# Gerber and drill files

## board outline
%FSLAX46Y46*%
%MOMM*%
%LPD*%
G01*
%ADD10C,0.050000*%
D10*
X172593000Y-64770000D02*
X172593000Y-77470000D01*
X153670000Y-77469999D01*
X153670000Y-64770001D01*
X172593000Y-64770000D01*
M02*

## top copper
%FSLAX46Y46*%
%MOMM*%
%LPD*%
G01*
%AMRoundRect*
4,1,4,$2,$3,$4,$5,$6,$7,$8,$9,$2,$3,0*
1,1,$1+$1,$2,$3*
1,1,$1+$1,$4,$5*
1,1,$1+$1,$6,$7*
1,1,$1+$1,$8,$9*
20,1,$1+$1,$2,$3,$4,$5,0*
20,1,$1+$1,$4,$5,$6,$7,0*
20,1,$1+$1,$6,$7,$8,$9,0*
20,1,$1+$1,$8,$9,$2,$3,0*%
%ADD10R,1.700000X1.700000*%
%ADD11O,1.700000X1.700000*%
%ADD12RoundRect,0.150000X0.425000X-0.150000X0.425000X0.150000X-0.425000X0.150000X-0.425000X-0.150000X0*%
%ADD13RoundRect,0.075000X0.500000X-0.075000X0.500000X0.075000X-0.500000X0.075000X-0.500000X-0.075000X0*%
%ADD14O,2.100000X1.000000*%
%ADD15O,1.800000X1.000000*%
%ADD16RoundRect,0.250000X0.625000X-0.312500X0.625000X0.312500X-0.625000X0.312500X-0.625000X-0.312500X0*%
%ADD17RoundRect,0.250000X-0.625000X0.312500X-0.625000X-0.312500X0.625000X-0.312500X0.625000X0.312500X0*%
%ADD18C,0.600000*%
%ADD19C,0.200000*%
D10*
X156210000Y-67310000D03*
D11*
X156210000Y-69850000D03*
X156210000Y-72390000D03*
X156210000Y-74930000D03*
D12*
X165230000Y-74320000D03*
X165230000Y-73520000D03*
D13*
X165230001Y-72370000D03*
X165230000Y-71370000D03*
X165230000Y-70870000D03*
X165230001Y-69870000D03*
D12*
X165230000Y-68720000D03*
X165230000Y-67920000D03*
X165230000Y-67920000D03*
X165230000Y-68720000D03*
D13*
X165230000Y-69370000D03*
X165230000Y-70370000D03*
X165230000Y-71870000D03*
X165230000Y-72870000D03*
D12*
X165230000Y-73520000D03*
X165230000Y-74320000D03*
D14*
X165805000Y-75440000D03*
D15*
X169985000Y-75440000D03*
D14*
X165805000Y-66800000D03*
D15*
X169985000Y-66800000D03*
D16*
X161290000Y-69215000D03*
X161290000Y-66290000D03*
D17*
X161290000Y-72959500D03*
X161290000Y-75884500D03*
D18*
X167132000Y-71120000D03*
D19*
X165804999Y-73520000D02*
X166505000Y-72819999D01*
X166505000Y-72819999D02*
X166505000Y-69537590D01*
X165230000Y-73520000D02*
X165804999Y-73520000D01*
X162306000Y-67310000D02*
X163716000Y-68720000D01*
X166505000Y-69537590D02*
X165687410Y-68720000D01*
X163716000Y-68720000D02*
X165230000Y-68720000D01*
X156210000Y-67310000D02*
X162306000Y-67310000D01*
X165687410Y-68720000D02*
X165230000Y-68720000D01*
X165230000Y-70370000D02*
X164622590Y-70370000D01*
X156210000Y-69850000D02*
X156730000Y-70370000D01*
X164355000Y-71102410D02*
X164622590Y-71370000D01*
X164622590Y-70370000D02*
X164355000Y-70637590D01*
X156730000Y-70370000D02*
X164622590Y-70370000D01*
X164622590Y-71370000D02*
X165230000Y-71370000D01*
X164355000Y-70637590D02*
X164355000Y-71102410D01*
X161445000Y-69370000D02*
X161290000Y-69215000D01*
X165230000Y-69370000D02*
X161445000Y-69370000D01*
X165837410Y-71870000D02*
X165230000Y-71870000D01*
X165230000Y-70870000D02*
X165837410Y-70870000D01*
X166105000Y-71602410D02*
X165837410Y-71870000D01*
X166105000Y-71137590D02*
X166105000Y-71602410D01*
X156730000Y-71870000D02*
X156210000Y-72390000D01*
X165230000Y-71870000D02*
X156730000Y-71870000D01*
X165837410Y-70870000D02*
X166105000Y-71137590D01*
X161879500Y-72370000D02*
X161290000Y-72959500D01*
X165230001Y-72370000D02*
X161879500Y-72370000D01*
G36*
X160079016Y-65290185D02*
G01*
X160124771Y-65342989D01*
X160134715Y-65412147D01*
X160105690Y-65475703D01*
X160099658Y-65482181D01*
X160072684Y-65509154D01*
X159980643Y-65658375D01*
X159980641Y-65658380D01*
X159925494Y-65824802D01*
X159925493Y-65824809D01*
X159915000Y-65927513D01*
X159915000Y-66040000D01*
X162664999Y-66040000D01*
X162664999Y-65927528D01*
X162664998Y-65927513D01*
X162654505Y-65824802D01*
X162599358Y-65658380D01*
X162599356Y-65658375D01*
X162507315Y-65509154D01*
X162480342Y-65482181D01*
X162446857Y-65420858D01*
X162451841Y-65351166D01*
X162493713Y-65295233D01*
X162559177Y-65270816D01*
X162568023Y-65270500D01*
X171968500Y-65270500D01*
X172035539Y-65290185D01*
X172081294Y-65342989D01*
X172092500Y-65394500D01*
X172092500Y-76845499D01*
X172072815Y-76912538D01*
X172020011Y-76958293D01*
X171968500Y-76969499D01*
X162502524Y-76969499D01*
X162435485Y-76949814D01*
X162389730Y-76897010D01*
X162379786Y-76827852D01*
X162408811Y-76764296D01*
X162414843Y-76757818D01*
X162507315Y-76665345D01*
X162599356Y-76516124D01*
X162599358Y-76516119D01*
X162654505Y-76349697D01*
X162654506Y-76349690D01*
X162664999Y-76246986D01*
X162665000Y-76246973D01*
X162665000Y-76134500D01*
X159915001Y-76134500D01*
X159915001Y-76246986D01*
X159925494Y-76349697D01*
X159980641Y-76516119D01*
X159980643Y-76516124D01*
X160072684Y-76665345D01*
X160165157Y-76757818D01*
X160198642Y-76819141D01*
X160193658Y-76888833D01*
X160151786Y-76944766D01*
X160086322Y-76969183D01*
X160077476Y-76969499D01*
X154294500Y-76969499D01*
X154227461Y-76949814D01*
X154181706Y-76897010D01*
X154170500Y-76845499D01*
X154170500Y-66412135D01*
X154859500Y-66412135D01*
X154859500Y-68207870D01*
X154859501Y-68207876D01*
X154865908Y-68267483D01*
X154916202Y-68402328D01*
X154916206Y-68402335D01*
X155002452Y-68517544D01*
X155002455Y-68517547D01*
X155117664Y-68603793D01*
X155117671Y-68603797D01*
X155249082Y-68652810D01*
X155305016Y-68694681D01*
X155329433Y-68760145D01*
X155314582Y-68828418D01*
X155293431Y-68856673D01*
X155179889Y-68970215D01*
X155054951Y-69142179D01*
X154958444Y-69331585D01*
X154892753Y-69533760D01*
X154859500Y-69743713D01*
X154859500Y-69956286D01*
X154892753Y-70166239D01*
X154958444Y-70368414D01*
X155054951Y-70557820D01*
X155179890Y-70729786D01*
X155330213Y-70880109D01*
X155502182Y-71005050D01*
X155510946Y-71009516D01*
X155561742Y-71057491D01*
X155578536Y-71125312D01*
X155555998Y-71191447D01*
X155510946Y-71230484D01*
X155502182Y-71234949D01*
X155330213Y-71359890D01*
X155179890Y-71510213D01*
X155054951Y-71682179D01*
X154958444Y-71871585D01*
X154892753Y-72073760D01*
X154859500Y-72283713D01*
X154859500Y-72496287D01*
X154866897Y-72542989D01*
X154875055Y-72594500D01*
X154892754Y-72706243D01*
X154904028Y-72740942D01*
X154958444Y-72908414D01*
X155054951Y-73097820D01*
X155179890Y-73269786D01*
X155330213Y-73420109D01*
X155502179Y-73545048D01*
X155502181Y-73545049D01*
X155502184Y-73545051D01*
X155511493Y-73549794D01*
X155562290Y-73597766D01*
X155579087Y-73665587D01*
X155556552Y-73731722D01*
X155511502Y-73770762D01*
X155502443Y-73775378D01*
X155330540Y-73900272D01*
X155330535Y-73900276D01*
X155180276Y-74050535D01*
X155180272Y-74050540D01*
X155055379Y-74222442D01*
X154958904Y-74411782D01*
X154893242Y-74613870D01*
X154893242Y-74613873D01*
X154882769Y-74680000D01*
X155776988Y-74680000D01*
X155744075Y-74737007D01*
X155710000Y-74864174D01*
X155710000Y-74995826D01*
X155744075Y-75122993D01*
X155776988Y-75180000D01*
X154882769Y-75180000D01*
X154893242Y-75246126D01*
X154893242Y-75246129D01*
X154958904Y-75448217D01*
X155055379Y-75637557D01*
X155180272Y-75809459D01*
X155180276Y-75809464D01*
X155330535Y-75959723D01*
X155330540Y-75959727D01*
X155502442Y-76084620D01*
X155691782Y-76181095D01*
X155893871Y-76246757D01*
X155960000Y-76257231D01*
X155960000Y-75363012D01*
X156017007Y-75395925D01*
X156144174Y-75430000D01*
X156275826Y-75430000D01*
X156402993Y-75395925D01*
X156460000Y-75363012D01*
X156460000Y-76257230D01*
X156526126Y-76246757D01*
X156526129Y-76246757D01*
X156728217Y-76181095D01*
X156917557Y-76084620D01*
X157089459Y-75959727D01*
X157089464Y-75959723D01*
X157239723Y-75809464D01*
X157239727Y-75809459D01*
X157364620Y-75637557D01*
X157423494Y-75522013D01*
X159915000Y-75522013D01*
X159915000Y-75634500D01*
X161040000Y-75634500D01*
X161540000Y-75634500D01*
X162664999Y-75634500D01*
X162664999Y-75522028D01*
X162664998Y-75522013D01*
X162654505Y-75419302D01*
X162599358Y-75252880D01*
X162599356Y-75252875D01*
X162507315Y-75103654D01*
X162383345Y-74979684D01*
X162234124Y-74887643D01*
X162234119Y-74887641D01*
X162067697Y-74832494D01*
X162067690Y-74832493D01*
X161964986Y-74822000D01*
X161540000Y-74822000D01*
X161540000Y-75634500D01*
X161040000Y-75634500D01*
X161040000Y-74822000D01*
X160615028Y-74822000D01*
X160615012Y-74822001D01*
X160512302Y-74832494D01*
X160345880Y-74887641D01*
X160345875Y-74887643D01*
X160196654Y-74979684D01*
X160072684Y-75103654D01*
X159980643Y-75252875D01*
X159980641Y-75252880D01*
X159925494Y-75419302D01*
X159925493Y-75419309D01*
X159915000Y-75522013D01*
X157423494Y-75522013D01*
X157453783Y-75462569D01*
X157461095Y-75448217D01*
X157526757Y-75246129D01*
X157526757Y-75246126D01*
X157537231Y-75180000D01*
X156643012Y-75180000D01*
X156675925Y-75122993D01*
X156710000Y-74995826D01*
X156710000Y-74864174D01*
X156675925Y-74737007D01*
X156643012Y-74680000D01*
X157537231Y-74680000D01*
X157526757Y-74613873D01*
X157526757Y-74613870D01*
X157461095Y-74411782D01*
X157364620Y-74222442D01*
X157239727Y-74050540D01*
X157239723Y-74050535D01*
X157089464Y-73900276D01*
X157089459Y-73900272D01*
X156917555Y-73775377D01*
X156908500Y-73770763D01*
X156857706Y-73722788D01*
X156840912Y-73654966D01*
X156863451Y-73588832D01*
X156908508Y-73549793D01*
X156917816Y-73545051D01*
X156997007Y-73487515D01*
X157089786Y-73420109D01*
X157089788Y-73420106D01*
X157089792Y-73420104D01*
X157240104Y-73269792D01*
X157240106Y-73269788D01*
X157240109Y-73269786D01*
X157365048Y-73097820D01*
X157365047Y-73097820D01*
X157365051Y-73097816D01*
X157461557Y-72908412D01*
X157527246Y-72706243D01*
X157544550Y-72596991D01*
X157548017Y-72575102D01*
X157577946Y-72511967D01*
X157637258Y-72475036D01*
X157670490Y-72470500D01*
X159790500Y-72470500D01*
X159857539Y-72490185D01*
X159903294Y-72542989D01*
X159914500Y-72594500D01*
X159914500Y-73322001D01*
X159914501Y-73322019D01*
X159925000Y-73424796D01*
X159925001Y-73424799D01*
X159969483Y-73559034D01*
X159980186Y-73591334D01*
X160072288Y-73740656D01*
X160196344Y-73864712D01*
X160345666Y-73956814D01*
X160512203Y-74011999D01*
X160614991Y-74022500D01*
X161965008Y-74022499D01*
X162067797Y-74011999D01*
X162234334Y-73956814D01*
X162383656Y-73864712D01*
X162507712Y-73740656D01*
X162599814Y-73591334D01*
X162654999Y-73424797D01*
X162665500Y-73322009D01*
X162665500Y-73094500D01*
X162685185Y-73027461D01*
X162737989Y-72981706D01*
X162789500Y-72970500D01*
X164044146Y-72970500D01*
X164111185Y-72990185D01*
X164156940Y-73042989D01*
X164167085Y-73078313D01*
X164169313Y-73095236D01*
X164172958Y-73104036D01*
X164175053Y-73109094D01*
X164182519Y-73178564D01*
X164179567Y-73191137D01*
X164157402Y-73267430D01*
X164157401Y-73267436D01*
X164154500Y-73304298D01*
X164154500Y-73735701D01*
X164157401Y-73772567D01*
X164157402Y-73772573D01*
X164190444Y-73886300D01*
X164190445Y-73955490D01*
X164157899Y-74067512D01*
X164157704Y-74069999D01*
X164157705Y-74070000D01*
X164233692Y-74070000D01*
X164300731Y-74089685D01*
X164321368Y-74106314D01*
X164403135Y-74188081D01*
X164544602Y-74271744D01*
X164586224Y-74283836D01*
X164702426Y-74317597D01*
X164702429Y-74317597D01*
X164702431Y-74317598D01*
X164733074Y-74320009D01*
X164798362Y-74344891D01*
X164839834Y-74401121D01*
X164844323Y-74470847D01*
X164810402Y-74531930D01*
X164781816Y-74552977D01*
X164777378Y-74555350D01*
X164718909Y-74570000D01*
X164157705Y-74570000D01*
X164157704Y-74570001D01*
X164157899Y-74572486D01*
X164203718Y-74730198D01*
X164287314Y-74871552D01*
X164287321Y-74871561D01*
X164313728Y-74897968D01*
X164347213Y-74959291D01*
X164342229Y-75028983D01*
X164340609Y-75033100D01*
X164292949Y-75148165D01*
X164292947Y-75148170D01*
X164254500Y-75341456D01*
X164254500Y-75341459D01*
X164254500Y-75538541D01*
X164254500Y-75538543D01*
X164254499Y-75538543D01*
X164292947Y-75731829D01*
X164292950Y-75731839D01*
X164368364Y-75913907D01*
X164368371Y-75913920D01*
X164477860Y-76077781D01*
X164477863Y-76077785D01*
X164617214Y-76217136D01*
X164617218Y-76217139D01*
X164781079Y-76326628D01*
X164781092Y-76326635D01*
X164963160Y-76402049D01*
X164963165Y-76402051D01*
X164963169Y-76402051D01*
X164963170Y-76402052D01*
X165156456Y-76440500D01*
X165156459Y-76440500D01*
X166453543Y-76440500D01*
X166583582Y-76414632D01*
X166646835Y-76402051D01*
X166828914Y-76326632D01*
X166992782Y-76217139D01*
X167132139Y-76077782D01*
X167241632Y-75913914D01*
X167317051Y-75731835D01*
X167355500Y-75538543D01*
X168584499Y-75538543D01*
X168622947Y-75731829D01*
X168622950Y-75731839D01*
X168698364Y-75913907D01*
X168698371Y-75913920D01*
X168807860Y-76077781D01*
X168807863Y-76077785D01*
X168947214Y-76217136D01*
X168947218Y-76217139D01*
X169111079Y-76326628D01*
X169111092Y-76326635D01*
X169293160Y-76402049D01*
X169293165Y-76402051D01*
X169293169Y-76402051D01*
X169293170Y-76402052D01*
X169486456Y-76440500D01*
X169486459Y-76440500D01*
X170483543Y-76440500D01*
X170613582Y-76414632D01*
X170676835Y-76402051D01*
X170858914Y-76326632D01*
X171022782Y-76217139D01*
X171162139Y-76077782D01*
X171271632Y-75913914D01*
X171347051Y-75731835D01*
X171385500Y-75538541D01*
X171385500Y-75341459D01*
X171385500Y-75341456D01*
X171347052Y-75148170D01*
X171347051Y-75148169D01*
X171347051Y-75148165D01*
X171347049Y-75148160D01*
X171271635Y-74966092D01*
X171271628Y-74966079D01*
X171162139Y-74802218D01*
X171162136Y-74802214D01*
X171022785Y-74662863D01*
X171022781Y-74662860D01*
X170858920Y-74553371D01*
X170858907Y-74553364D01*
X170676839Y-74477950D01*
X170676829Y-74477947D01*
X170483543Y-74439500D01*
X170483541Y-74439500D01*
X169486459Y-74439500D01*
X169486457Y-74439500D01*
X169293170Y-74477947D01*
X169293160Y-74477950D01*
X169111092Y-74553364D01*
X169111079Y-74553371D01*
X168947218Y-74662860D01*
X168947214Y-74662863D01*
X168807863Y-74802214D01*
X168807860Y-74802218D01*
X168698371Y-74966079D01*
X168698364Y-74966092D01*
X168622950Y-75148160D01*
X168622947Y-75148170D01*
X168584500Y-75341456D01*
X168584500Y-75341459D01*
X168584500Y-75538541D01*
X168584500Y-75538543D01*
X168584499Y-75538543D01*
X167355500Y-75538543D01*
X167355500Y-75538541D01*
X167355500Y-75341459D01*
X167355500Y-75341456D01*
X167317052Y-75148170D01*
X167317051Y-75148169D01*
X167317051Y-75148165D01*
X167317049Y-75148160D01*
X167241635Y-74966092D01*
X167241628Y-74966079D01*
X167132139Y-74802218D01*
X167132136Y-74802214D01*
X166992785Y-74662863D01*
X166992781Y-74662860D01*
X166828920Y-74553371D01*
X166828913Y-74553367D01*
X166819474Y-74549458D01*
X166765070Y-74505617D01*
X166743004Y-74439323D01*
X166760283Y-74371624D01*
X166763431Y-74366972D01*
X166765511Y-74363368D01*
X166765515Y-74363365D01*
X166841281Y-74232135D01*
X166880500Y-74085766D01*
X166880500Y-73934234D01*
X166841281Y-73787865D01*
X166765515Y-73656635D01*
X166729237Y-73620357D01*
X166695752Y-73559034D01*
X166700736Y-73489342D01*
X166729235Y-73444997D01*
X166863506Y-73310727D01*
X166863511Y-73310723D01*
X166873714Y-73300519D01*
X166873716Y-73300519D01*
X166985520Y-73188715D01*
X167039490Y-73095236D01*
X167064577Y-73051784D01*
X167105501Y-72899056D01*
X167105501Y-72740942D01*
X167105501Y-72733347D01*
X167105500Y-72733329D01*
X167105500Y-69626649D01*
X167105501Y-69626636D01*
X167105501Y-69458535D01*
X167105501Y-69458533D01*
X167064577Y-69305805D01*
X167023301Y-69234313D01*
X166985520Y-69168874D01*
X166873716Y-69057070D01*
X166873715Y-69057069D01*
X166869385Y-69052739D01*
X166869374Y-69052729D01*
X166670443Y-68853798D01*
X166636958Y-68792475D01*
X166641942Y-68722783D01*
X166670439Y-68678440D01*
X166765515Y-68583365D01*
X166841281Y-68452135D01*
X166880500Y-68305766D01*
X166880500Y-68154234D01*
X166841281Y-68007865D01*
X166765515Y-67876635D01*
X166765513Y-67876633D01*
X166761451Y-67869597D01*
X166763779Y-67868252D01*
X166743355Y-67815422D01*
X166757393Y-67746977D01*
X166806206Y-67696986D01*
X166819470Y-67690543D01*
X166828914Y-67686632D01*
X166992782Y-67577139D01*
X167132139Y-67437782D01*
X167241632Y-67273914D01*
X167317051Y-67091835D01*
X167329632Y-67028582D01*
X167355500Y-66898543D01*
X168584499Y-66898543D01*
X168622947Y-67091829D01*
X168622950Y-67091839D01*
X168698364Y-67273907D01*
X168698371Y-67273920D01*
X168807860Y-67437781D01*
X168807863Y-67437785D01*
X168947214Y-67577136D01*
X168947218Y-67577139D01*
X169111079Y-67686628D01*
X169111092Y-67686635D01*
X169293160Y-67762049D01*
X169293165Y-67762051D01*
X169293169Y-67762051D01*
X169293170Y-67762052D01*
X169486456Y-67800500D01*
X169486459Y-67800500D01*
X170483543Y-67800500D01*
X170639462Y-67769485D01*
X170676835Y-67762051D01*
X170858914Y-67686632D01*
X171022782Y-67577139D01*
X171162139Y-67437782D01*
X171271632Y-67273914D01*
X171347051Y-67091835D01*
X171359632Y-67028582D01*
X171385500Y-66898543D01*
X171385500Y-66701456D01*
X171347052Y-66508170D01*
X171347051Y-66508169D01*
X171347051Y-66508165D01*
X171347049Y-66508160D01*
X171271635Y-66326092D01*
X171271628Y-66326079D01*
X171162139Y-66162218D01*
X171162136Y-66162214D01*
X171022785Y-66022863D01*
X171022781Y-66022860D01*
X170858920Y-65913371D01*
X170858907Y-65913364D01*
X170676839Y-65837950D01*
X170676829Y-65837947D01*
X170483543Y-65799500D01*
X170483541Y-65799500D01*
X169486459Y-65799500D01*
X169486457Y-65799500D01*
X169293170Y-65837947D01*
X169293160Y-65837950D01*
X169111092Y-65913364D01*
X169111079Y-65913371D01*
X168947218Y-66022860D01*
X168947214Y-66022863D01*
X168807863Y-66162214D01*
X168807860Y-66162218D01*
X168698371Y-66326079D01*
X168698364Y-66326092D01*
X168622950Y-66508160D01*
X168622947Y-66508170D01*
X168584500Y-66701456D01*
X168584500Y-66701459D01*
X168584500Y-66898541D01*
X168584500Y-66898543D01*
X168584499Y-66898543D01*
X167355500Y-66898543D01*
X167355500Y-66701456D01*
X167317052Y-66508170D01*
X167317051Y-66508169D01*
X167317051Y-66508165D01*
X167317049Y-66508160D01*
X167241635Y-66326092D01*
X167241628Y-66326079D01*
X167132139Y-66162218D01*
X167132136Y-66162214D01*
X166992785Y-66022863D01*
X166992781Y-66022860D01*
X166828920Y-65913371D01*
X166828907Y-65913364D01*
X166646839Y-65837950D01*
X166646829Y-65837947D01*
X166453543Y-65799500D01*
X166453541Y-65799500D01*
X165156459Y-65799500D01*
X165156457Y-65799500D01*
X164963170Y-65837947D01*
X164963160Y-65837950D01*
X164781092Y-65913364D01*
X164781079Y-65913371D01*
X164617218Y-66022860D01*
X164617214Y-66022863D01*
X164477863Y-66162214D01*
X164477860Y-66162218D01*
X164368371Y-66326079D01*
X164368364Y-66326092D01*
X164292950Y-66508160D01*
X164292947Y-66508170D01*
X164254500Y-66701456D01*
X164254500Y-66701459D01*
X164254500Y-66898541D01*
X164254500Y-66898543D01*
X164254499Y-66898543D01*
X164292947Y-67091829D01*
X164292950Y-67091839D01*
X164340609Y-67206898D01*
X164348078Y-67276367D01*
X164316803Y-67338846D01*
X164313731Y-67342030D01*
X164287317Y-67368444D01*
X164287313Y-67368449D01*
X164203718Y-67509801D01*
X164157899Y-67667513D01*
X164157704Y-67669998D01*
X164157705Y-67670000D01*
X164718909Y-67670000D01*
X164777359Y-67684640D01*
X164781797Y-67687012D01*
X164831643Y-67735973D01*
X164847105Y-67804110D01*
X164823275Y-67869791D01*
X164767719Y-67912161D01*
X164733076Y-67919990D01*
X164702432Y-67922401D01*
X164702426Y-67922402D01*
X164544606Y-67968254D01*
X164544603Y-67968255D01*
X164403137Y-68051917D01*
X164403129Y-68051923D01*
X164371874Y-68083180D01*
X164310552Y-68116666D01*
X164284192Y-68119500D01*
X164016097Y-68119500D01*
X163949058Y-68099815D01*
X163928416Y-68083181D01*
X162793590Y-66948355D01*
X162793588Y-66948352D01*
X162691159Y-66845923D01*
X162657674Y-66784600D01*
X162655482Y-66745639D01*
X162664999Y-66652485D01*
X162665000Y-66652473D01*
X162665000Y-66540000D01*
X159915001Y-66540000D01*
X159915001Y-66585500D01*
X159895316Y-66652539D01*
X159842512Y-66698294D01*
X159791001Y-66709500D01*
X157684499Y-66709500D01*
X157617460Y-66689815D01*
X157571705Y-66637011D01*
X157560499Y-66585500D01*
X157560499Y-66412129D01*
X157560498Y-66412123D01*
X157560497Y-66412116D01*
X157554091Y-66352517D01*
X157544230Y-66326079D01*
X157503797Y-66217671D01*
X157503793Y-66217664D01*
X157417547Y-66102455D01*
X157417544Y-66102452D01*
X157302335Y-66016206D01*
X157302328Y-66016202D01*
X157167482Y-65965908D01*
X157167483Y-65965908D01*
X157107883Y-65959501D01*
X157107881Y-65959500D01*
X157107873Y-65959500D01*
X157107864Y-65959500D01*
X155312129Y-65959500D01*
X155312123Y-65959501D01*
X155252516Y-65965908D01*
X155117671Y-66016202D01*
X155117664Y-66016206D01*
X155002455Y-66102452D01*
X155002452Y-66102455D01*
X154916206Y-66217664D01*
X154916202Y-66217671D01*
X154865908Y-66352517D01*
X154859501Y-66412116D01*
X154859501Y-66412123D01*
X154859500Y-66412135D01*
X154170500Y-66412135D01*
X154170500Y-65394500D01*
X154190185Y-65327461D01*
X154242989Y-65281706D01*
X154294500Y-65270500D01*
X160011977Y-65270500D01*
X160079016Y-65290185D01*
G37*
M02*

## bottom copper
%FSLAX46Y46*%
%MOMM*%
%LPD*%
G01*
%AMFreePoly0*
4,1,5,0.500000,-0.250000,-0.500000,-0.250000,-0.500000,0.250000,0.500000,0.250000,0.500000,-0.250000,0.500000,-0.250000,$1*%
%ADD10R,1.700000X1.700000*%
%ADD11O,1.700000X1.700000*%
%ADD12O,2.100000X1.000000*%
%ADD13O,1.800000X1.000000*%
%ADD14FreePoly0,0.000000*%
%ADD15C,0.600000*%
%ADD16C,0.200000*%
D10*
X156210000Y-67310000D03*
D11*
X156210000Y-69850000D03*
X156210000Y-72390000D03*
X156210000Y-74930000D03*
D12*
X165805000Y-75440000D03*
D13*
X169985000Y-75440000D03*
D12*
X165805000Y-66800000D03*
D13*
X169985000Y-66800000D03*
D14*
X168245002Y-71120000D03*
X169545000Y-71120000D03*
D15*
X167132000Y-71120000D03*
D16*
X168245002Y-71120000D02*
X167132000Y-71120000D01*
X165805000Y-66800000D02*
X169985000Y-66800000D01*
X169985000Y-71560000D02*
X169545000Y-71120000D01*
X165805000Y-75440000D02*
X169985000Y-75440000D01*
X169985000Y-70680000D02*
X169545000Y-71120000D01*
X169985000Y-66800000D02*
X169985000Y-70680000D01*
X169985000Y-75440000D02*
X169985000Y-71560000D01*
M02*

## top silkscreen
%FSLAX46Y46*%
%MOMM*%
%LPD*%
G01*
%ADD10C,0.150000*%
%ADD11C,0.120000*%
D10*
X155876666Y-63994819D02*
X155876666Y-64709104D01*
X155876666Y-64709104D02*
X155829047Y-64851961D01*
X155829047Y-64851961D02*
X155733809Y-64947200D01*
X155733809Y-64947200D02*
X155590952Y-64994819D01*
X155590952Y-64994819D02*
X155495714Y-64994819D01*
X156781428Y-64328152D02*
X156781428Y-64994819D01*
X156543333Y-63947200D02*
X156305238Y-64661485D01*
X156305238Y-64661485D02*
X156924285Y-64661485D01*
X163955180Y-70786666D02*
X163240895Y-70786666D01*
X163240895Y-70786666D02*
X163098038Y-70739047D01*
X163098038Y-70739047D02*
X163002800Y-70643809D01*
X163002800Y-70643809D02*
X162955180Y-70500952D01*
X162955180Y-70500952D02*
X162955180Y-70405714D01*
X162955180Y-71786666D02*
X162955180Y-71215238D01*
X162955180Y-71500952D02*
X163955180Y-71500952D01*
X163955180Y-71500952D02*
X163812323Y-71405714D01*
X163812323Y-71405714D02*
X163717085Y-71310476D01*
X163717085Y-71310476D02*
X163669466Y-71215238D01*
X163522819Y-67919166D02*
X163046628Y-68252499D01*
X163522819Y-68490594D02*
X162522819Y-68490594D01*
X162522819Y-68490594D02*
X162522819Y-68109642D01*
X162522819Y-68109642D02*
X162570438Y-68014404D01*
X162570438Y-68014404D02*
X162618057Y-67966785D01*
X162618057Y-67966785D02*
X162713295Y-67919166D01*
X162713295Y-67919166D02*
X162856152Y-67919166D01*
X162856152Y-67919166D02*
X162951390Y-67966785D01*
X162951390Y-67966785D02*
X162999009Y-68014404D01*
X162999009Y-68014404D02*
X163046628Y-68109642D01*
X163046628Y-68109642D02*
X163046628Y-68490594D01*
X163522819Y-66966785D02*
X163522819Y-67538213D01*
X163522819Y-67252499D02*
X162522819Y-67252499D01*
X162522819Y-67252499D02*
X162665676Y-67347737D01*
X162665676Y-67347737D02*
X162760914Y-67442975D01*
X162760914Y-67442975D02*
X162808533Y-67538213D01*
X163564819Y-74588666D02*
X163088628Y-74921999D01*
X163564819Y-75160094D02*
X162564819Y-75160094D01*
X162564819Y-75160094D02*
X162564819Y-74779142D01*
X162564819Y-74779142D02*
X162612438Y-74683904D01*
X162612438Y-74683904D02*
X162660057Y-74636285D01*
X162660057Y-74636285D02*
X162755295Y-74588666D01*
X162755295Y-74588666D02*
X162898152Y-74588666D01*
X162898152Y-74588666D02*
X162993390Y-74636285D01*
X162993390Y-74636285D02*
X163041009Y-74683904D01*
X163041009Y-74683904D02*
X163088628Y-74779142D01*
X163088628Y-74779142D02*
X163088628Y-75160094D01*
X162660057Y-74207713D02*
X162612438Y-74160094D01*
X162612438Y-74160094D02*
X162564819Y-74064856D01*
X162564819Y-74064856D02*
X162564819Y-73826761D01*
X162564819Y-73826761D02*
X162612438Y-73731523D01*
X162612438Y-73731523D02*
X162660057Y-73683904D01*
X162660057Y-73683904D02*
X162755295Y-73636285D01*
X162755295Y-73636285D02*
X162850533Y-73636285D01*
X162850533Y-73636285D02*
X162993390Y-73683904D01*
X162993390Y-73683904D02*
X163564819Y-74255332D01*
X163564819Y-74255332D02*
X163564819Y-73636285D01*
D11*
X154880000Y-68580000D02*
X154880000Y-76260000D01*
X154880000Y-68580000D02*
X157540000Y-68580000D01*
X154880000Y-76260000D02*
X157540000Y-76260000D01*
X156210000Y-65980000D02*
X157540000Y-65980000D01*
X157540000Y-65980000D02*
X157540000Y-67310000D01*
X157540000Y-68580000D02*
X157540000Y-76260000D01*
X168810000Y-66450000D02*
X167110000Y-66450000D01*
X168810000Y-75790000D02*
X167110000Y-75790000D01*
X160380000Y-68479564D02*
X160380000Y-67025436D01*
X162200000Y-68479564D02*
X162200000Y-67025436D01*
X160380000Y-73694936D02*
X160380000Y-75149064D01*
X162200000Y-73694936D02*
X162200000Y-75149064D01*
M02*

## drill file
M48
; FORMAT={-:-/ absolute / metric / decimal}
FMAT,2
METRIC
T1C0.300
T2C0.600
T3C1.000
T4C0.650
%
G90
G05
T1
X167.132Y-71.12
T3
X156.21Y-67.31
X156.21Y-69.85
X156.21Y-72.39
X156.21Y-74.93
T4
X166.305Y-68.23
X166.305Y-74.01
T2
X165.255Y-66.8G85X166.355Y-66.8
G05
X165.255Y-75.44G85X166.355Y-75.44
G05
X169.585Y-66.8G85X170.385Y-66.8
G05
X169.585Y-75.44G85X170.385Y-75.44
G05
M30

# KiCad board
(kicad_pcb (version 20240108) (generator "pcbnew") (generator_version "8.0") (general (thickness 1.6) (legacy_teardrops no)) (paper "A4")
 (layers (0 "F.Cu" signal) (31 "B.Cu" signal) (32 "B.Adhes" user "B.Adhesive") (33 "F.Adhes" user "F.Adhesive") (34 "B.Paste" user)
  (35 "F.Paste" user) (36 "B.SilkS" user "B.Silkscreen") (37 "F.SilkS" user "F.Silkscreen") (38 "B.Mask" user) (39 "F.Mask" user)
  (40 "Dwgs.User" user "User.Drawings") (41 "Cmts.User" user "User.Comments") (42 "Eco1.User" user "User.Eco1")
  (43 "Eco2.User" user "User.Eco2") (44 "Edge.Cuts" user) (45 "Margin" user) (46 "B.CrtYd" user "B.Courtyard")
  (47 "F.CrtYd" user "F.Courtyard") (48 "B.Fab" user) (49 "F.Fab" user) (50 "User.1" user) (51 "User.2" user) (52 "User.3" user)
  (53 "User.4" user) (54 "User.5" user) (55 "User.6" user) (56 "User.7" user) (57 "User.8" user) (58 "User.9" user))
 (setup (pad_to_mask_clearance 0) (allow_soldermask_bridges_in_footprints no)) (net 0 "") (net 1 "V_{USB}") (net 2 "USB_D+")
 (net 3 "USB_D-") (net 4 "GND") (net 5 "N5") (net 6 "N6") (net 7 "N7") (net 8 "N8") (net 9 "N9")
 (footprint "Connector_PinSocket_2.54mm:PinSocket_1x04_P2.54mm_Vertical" (layer "F.Cu") (at 156.21 67.31)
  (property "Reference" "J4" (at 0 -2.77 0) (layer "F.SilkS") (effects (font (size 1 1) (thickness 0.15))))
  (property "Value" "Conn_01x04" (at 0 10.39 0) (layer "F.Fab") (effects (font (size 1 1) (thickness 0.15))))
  (fp_line (start -1.33 1.27) (end -1.33 8.95) (stroke (width 0.12) (type solid)) (layer "F.SilkS"))
  (fp_line (start -1.33 1.27) (end 1.33 1.27) (stroke (width 0.12) (type solid)) (layer "F.SilkS"))
  (fp_line (start -1.33 8.95) (end 1.33 8.95) (stroke (width 0.12) (type solid)) (layer "F.SilkS"))
  (fp_line (start 0 -1.33) (end 1.33 -1.33) (stroke (width 0.12) (type solid)) (layer "F.SilkS"))
  (fp_line (start 1.33 -1.33) (end 1.33 0) (stroke (width 0.12) (type solid)) (layer "F.SilkS"))
  (fp_line (start 1.33 1.27) (end 1.33 8.95) (stroke (width 0.12) (type solid)) (layer "F.SilkS"))
  (pad "1" thru_hole rect (at 0 0) (size 1.7 1.7) (drill 1) (layers "*.Cu" "*.Mask") (remove_unused_layers no) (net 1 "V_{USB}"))
  (pad "2" thru_hole oval (at 0 2.54) (size 1.7 1.7) (drill 1) (layers "*.Cu" "*.Mask") (remove_unused_layers no) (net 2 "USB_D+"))
  (pad "3" thru_hole oval (at 0 5.08) (size 1.7 1.7) (drill 1) (layers "*.Cu" "*.Mask") (remove_unused_layers no) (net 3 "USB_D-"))
  (pad "4" thru_hole oval (at 0 7.62) (size 1.7 1.7) (drill 1) (layers "*.Cu" "*.Mask") (remove_unused_layers no) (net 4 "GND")))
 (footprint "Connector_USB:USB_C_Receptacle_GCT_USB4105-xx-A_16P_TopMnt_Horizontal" (layer "F.Cu") (at 168.91 71.12 90)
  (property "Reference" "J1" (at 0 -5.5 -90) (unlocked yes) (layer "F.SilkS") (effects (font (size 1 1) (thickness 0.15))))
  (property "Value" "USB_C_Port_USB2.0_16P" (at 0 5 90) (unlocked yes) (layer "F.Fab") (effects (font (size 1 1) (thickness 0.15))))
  (fp_line (start 4.67 -0.1) (end 4.67 -1.8) (stroke (width 0.12) (type solid)) (layer "F.SilkS"))
  (fp_line (start -4.67 -0.1) (end -4.67 -1.8) (stroke (width 0.12) (type solid)) (layer "F.SilkS"))
  (pad "" np_thru_hole circle (at -2.89 -2.605 90) (size 0.65 0.65) (drill 0.65) (layers "F&B.Cu" "*.Mask"))
  (pad "" np_thru_hole circle (at 2.89 -2.605 90) (size 0.65 0.65) (drill 0.65) (layers "F&B.Cu" "*.Mask"))
  (pad "A1" smd roundrect (at -3.2 -3.68 90) (size 0.6 1.15) (layers "F.Cu" "F.Paste" "F.Mask") (roundrect_rratio 0.25) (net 4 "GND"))
  (pad "A4" smd roundrect (at -2.4 -3.68 90) (size 0.6 1.15) (layers "F.Cu" "F.Paste" "F.Mask") (roundrect_rratio 0.25) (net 1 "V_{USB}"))
  (pad "A5" smd roundrect (at -1.25 -3.679999 90) (size 0.3 1.15) (layers "F.Cu" "F.Paste" "F.Mask") (roundrect_rratio 0.25) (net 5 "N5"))
  (pad "A6" smd roundrect (at -0.25 -3.68 90) (size 0.3 1.15) (layers "F.Cu" "F.Paste" "F.Mask") (roundrect_rratio 0.25) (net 2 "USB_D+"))
  (pad "A7" smd roundrect (at 0.25 -3.68 90) (size 0.3 1.15) (layers "F.Cu" "F.Paste" "F.Mask") (roundrect_rratio 0.25) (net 3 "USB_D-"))
  (pad "A8" smd roundrect (at 1.25 -3.679999 90) (size 0.3 1.15) (layers "F.Cu" "F.Paste" "F.Mask") (roundrect_rratio 0.25) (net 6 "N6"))
  (pad "A9" smd roundrect (at 2.4 -3.68 90) (size 0.6 1.15) (layers "F.Cu" "F.Paste" "F.Mask") (roundrect_rratio 0.25) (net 1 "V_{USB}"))
  (pad "A12" smd roundrect (at 3.2 -3.68 90) (size 0.6 1.15) (layers "F.Cu" "F.Paste" "F.Mask") (roundrect_rratio 0.25) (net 4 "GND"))
  (pad "B1" smd roundrect (at 3.2 -3.68 90) (size 0.6 1.15) (layers "F.Cu" "F.Paste" "F.Mask") (roundrect_rratio 0.25) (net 4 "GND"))
  (pad "B4" smd roundrect (at 2.4 -3.68 90) (size 0.6 1.15) (layers "F.Cu" "F.Paste" "F.Mask") (roundrect_rratio 0.25) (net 1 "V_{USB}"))
  (pad "B5" smd roundrect (at 1.75 -3.68 90) (size 0.3 1.15) (layers "F.Cu" "F.Paste" "F.Mask") (roundrect_rratio 0.25) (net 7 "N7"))
  (pad "B6" smd roundrect (at 0.75 -3.68 90) (size 0.3 1.15) (layers "F.Cu" "F.Paste" "F.Mask") (roundrect_rratio 0.25) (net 2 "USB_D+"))
  (pad "B7" smd roundrect (at -0.75 -3.68 90) (size 0.3 1.15) (layers "F.Cu" "F.Paste" "F.Mask") (roundrect_rratio 0.25) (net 3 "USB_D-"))
  (pad "B8" smd roundrect (at -1.75 -3.68 90) (size 0.3 1.15) (layers "F.Cu" "F.Paste" "F.Mask") (roundrect_rratio 0.25) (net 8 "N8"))
  (pad "B9" smd roundrect (at -2.4 -3.68 90) (size 0.6 1.15) (layers "F.Cu" "F.Paste" "F.Mask") (roundrect_rratio 0.25) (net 1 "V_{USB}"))
  (pad "B12" smd roundrect (at -3.2 -3.68 90) (size 0.6 1.15) (layers "F.Cu" "F.Paste" "F.Mask") (roundrect_rratio 0.25) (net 4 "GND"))
  (pad "S1" thru_hole oval (at -4.32 -3.105 90) (size 1 2.1) (drill oval 0.6 1.7) (layers "*.Cu" "*.Mask" "F.Paste")
   (remove_unused_layers no) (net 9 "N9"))
  (pad "S1" thru_hole oval (at -4.32 1.075 90) (size 1 1.8) (drill oval 0.6 1.4) (layers "*.Cu" "*.Mask" "F.Paste")
   (remove_unused_layers no) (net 9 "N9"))
  (pad "S1" thru_hole oval (at 4.32 -3.105 90) (size 1 2.1) (drill oval 0.6 1.7) (layers "*.Cu" "*.Mask" "F.Paste")
   (remove_unused_layers no) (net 9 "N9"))
  (pad "S1" thru_hole oval (at 4.32 1.075 90) (size 1 1.8) (drill oval 0.6 1.4) (layers "*.Cu" "*.Mask" "F.Paste") (remove_unused_layers no)
   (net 9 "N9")))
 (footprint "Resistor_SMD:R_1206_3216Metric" (layer "F.Cu") (at 161.29 67.7525 90)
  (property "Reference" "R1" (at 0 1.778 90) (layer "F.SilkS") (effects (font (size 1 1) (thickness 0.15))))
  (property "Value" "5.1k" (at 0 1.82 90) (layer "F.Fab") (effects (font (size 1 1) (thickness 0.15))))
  (fp_line (start -0.727064 -0.91) (end 0.727064 -0.91) (stroke (width 0.12) (type solid)) (layer "F.SilkS"))
  (fp_line (start -0.727064 0.91) (end 0.727064 0.91) (stroke (width 0.12) (type solid)) (layer "F.SilkS"))
  (pad "1" smd roundrect (at -1.4625 0 90) (size 1.125 1.75) (layers "F.Cu" "F.Paste" "F.Mask") (roundrect_rratio 0.222222) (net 7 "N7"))
  (pad "2" smd roundrect (at 1.4625 0 90) (size 1.125 1.75) (layers "F.Cu" "F.Paste" "F.Mask") (roundrect_rratio 0.222222) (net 4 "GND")))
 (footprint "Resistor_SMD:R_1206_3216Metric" (layer "F.Cu") (at 161.29 74.422 -90)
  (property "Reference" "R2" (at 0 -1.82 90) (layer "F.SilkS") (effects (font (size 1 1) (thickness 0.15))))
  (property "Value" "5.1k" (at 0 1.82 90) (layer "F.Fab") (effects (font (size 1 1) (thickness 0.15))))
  (fp_line (start -0.727064 0.91) (end 0.727064 0.91) (stroke (width 0.12) (type solid)) (layer "F.SilkS"))
  (fp_line (start -0.727064 -0.91) (end 0.727064 -0.91) (stroke (width 0.12) (type solid)) (layer "F.SilkS"))
  (pad "1" smd roundrect (at -1.4625 0 270) (size 1.125 1.75) (layers "F.Cu" "F.Paste" "F.Mask") (roundrect_rratio 0.222222) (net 5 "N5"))
  (pad "2" smd roundrect (at 1.4625 0 270) (size 1.125 1.75) (layers "F.Cu" "F.Paste" "F.Mask") (roundrect_rratio 0.222222) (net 4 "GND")))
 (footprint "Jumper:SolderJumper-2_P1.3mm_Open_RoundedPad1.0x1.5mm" (layer "B.Cu") (at 168.895001 71.12)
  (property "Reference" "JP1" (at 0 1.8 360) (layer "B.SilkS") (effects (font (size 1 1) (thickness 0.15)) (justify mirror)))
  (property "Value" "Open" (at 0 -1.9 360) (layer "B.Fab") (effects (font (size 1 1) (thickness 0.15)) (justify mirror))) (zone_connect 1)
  (pad "1" smd custom (at -0.649999 0) (size 1 0.5) (layers "B.Cu" "B.Mask") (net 4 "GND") (zone_connect 2) (thermal_bridge_angle 45)
   (options (clearance outline) (anchor rect)) (primitives))
  (pad "2" smd custom (at 0.649999 0) (size 1 0.5) (layers "B.Cu" "B.Mask") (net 9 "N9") (zone_connect 2) (thermal_bridge_angle 45)
   (options (clearance outline) (anchor rect)) (primitives)))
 (gr_poly
  (pts (xy 172.593 64.77) (xy 172.593 77.47) (xy 153.67 77.469999) (xy 153.67 64.770001)) (stroke (width 0.05) (type default)) (fill none)
  (layer "Edge.Cuts"))
 (segment (start 165.804999 73.52) (end 166.505 72.819999) (width 0.2) (layer "F.Cu") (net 1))
 (segment (start 166.505 72.819999) (end 166.505 69.53759) (width 0.2) (layer "F.Cu") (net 1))
 (segment (start 165.23 73.52) (end 165.804999 73.52) (width 0.2) (layer "F.Cu") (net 1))
 (segment (start 162.306 67.31) (end 163.716 68.72) (width 0.2) (layer "F.Cu") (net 1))
 (segment (start 166.505 69.53759) (end 165.68741 68.72) (width 0.2) (layer "F.Cu") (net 1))
 (segment (start 163.716 68.72) (end 165.23 68.72) (width 0.2) (layer "F.Cu") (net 1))
 (segment (start 156.21 67.31) (end 162.306 67.31) (width 0.2) (layer "F.Cu") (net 1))
 (segment (start 165.68741 68.72) (end 165.23 68.72) (width 0.2) (layer "F.Cu") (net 1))
 (via (at 167.132 71.12) (size 0.6) (drill 0.3) (layers "F.Cu" "B.Cu") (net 4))
 (segment (start 168.245002 71.12) (end 167.132 71.12) (width 0.2) (layer "B.Cu") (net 4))
 (segment (start 165.805 66.8) (end 169.985 66.8) (width 0.2) (layer "B.Cu") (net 9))
 (segment (start 169.985 71.56) (end 169.545 71.12) (width 0.2) (layer "B.Cu") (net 9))
 (segment (start 165.805 75.44) (end 169.985 75.44) (width 0.2) (layer "B.Cu") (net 9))
 (segment (start 169.985 70.68) (end 169.545 71.12) (width 0.2) (layer "B.Cu") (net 9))
 (segment (start 169.985 66.8) (end 169.985 70.68) (width 0.2) (layer "B.Cu") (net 9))
 (segment (start 169.985 75.44) (end 169.985 71.56) (width 0.2) (layer "B.Cu") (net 9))
 (segment (start 165.23 70.37) (end 164.62259 70.37) (width 0.2) (layer "F.Cu") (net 2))
 (segment (start 156.21 69.85) (end 156.73 70.37) (width 0.2) (layer "F.Cu") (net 2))
 (segment (start 164.355 71.10241) (end 164.62259 71.37) (width 0.2) (layer "F.Cu") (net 2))
 (segment (start 164.62259 70.37) (end 164.355 70.63759) (width 0.2) (layer "F.Cu") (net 2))
 (segment (start 156.73 70.37) (end 164.62259 70.37) (width 0.2) (layer "F.Cu") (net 2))
 (segment (start 164.62259 71.37) (end 165.23 71.37) (width 0.2) (layer "F.Cu") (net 2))
 (segment (start 164.355 70.63759) (end 164.355 71.10241) (width 0.2) (layer "F.Cu") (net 2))
 (segment (start 161.445 69.37) (end 161.29 69.215) (width 0.2) (layer "F.Cu") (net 7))
 (segment (start 165.23 69.37) (end 161.445 69.37) (width 0.2) (layer "F.Cu") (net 7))
 (segment (start 165.83741 71.87) (end 165.23 71.87) (width 0.2) (layer "F.Cu") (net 3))
 (segment (start 165.23 70.87) (end 165.83741 70.87) (width 0.2) (layer "F.Cu") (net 3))
 (segment (start 166.105 71.60241) (end 165.83741 71.87) (width 0.2) (layer "F.Cu") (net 3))
 (segment (start 166.105 71.13759) (end 166.105 71.60241) (width 0.2) (layer "F.Cu") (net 3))
 (segment (start 156.73 71.87) (end 156.21 72.39) (width 0.2) (layer "F.Cu") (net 3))
 (segment (start 165.23 71.87) (end 156.73 71.87) (width 0.2) (layer "F.Cu") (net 3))
 (segment (start 165.83741 70.87) (end 166.105 71.13759) (width 0.2) (layer "F.Cu") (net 3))
 (segment (start 161.8795 72.37) (end 161.29 72.9595) (width 0.2) (layer "F.Cu") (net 5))
 (segment (start 165.230001 72.37) (end 161.8795 72.37) (width 0.2) (layer "F.Cu") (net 5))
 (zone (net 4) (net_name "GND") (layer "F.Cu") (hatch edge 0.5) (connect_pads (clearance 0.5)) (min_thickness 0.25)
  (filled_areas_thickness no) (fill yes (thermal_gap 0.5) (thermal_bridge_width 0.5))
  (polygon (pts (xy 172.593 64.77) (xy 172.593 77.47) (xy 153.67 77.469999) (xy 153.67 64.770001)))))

